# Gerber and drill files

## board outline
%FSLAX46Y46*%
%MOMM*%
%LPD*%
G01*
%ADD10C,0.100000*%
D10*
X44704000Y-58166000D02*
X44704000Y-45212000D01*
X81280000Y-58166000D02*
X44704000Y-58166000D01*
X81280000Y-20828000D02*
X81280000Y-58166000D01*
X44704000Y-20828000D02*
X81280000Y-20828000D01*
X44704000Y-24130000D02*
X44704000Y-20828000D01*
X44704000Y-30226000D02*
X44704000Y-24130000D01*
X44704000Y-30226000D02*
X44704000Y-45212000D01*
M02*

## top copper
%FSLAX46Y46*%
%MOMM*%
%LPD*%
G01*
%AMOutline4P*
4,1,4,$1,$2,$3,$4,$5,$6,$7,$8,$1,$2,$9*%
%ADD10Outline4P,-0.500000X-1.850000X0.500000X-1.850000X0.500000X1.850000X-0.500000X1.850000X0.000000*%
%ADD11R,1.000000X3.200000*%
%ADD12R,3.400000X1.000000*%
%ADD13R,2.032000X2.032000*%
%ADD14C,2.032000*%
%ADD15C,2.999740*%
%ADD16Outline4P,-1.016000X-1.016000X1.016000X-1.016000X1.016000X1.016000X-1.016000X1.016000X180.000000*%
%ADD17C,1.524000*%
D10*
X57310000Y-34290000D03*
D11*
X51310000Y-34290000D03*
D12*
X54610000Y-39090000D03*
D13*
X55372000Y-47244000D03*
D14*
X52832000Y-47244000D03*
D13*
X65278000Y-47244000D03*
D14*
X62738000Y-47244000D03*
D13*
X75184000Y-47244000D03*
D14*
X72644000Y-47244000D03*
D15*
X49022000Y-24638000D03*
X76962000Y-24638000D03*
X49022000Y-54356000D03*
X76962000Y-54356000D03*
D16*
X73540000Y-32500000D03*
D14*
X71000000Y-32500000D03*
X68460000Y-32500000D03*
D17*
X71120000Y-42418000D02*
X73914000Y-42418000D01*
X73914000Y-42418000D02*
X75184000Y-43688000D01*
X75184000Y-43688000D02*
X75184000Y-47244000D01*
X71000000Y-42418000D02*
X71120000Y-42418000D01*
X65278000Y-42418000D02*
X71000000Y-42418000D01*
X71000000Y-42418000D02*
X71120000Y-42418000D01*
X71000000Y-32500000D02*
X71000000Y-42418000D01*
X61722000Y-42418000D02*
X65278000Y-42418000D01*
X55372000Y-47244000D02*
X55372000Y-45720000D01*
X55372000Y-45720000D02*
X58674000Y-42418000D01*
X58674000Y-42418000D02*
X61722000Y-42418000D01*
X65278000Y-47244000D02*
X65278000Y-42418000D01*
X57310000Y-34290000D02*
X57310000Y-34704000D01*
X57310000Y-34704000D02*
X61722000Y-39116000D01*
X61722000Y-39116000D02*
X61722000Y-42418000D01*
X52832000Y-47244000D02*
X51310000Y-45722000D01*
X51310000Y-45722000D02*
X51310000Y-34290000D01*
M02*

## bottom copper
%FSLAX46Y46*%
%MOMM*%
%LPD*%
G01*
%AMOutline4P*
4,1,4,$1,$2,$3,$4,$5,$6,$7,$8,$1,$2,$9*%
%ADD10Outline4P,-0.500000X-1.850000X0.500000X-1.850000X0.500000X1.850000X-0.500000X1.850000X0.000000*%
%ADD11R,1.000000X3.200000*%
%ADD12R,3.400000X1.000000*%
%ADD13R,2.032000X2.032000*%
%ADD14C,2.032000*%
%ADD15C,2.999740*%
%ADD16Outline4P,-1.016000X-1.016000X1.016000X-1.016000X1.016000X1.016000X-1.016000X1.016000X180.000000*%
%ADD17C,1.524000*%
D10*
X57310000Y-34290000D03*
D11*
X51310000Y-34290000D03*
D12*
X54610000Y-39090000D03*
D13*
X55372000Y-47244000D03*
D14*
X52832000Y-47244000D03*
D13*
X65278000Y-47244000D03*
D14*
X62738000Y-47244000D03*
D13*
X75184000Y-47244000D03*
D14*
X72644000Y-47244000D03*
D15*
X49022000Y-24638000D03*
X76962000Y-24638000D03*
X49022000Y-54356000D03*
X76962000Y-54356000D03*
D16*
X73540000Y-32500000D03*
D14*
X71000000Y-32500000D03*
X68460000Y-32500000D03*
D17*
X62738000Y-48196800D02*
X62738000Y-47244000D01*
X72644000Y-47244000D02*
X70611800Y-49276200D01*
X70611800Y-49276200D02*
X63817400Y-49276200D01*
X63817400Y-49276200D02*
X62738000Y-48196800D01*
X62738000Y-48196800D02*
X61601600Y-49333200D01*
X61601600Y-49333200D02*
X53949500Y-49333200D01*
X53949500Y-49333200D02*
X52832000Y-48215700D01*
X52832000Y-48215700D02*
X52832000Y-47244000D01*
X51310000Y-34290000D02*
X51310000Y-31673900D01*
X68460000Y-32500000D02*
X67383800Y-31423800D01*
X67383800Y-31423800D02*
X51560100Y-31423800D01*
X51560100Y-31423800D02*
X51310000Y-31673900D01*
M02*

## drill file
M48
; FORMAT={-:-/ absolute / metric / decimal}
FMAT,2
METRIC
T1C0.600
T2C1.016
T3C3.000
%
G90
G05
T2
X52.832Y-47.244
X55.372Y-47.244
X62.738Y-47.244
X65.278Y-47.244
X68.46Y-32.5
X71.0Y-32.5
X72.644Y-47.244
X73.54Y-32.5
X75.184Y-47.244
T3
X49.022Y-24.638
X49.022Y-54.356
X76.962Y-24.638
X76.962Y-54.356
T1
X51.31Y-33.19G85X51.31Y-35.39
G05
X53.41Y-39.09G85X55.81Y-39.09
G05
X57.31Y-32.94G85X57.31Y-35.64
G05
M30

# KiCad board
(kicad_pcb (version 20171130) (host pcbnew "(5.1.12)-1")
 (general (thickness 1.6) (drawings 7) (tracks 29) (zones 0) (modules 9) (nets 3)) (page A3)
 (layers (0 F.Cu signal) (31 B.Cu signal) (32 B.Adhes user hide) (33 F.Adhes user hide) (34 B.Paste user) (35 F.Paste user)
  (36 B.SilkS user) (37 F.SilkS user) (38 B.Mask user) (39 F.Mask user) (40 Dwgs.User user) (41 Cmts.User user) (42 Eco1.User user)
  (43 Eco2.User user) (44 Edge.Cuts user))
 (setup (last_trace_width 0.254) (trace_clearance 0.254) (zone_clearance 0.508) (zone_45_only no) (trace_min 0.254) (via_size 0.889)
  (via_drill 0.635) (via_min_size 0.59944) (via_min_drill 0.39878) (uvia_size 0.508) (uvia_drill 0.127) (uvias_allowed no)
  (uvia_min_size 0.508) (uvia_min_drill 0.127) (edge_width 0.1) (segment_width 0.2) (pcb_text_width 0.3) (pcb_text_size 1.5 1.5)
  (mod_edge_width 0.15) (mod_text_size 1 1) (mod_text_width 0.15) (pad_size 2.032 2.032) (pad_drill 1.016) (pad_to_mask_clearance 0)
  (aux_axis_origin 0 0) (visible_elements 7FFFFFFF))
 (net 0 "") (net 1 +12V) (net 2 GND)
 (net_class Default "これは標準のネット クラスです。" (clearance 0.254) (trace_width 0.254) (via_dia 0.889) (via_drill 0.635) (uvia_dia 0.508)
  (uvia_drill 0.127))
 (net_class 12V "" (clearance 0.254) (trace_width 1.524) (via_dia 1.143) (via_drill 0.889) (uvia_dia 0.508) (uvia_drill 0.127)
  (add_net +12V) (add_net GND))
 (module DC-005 (layer F.Cu) (at 54.61 34.29)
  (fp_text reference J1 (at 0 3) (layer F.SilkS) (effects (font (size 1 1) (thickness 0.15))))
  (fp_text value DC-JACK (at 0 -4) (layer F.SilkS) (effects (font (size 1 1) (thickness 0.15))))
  (pad 1 thru_hole trapezoid (at 2.7 0) (size 1 3.7) (drill oval 0.6 3.3) (layers *.Cu *.Mask F.SilkS) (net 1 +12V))
  (pad 2 thru_hole rect (at -3.3 0) (size 1 3.2) (drill oval 0.6 2.8) (layers *.Cu *.Mask F.SilkS) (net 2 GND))
  (pad 3 thru_hole rect (at 0 4.8) (size 3.4 1) (drill oval 3 0.6) (layers *.Cu *.Mask F.SilkS)))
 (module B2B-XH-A (layer F.Cu) (at 54.102 47.244 180)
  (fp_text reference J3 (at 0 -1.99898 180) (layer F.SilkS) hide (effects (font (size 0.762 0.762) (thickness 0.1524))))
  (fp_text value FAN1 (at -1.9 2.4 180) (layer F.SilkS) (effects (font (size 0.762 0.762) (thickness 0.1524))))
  (pad 1 thru_hole rect (at -1.27 0 180) (size 2.032 2.032) (drill 1.016) (layers *.Cu *.Mask F.SilkS) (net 1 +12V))
  (pad 2 thru_hole circle (at 1.27 0 180) (size 2.032 2.032) (drill 1.016) (layers *.Cu *.Mask F.SilkS) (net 2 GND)))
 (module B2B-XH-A (layer F.Cu) (at 64.008 47.244 180)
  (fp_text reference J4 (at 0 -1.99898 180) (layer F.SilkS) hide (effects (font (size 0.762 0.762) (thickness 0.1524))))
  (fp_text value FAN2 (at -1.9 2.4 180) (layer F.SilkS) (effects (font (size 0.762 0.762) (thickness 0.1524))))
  (pad 1 thru_hole rect (at -1.27 0 180) (size 2.032 2.032) (drill 1.016) (layers *.Cu *.Mask F.SilkS) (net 1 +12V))
  (pad 2 thru_hole circle (at 1.27 0 180) (size 2.032 2.032) (drill 1.016) (layers *.Cu *.Mask F.SilkS) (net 2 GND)))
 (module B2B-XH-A (layer F.Cu) (at 73.914 47.244 180)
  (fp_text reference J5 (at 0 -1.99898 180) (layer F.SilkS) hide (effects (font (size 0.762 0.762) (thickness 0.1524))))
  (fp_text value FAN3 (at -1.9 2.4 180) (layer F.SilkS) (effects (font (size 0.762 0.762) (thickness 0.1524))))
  (pad 1 thru_hole rect (at -1.27 0 180) (size 2.032 2.032) (drill 1.016) (layers *.Cu *.Mask F.SilkS) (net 1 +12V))
  (pad 2 thru_hole circle (at 1.27 0 180) (size 2.032 2.032) (drill 1.016) (layers *.Cu *.Mask F.SilkS) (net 2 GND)))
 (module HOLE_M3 (layer F.Cu) (at 49.022 24.638)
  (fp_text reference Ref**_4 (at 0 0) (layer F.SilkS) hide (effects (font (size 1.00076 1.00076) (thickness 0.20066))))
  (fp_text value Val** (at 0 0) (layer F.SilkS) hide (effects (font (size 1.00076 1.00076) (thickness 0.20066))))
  (pad "" thru_hole circle (at 0 0) (size 2.99974 2.99974) (drill 2.99974) (layers *.Cu *.Mask F.SilkS) (clearance 1.50114)))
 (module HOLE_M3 (layer F.Cu) (at 76.962 24.638)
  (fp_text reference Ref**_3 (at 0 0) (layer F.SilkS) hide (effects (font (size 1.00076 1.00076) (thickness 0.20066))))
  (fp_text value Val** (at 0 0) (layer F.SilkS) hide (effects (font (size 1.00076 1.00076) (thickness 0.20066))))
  (pad "" thru_hole circle (at 0 0) (size 2.99974 2.99974) (drill 2.99974) (layers *.Cu *.Mask F.SilkS) (clearance 1.50114)))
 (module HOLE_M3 (layer F.Cu) (at 49.022 54.356)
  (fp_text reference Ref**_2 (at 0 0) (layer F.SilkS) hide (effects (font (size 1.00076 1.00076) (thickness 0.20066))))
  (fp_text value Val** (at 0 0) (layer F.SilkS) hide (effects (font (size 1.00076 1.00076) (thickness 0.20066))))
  (pad "" thru_hole circle (at 0 0) (size 2.99974 2.99974) (drill 2.99974) (layers *.Cu *.Mask F.SilkS) (clearance 1.50114)))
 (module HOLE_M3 (layer F.Cu) (at 76.962 54.356)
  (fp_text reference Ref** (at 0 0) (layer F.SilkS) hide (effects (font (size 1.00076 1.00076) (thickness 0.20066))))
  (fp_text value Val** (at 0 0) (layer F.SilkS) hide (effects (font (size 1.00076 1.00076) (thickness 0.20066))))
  (pad "" thru_hole circle (at 0 0) (size 2.99974 2.99974) (drill 2.99974) (layers *.Cu *.Mask F.SilkS) (clearance 1.50114)))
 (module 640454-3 (layer F.Cu) (at 71 32.5 180)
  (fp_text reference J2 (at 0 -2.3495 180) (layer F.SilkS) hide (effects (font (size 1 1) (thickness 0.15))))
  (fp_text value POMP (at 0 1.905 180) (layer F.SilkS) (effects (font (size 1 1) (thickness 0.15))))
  (pad 1 thru_hole trapezoid (at -2.54 0 180) (size 2.032 2.032) (drill 1.016) (layers *.Cu *.Mask F.SilkS))
  (pad 2 thru_hole circle (at 0 0 180) (size 2.032 2.032) (drill 1.016) (layers *.Cu *.Mask F.SilkS) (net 1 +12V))
  (pad 3 thru_hole circle (at 2.54 0 180) (size 2.032 2.032) (drill 1.016) (layers *.Cu *.Mask F.SilkS) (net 2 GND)))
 (gr_line (start 44.704 58.166) (end 44.704 45.212) (angle 90) (layer Edge.Cuts) (width 0.1))
 (gr_line (start 81.28 58.166) (end 44.704 58.166) (angle 90) (layer Edge.Cuts) (width 0.1))
 (gr_line (start 81.28 20.828) (end 81.28 58.166) (angle 90) (layer Edge.Cuts) (width 0.1))
 (gr_line (start 44.704 20.828) (end 81.28 20.828) (angle 90) (layer Edge.Cuts) (width 0.1))
 (gr_line (start 44.704 24.13) (end 44.704 20.828) (angle 90) (layer Edge.Cuts) (width 0.1))
 (gr_line (start 44.704 30.226) (end 44.704 24.13) (angle 90) (layer Edge.Cuts) (width 0.1))
 (gr_line (start 44.704 30.226) (end 44.704 45.212) (angle 90) (layer Edge.Cuts) (width 0.1))
 (segment (start 71.12 42.418) (end 73.914 42.418) (width 1.524) (layer F.Cu) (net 1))
 (segment (start 73.914 42.418) (end 75.184 43.688) (width 1.524) (layer F.Cu) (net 1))
 (segment (start 75.184 43.688) (end 75.184 47.244) (width 1.524) (layer F.Cu) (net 1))
 (segment (start 71 42.418) (end 71.12 42.418) (width 1.524) (layer F.Cu) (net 1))
 (segment (start 65.278 42.418) (end 71 42.418) (width 1.524) (layer F.Cu) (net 1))
 (segment (start 71 42.418) (end 71.12 42.418) (width 1.524) (layer F.Cu) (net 1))
 (segment (start 71 32.5) (end 71 42.418) (width 1.524) (layer F.Cu) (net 1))
 (segment (start 61.722 42.418) (end 65.278 42.418) (width 1.524) (layer F.Cu) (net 1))
 (segment (start 55.372 47.244) (end 55.372 45.72) (width 1.524) (layer F.Cu) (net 1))
 (segment (start 55.372 45.72) (end 58.674 42.418) (width 1.524) (layer F.Cu) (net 1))
 (segment (start 58.674 42.418) (end 61.722 42.418) (width 1.524) (layer F.Cu) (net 1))
 (segment (start 65.278 47.244) (end 65.278 42.418) (width 1.524) (layer F.Cu) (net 1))
 (segment (start 57.31 34.29) (end 57.31 34.704) (width 1.524) (layer F.Cu) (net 1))
 (segment (start 57.31 34.704) (end 61.722 39.116) (width 1.524) (layer F.Cu) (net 1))
 (segment (start 61.722 39.116) (end 61.722 42.418) (width 1.524) (layer F.Cu) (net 1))
 (segment (start 52.832 47.244) (end 51.31 45.722) (width 1.524) (layer F.Cu) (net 2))
 (segment (start 51.31 45.722) (end 51.31 34.29) (width 1.524) (layer F.Cu) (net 2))
 (segment (start 62.738 48.1968) (end 62.738 47.244) (width 1.524) (layer B.Cu) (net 2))
 (segment (start 72.644 47.244) (end 70.6118 49.2762) (width 1.524) (layer B.Cu) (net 2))
 (segment (start 70.6118 49.2762) (end 63.8174 49.2762) (width 1.524) (layer B.Cu) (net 2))
 (segment (start 63.8174 49.2762) (end 62.738 48.1968) (width 1.524) (layer B.Cu) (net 2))
 (segment (start 62.738 48.1968) (end 61.6016 49.3332) (width 1.524) (layer B.Cu) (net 2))
 (segment (start 61.6016 49.3332) (end 53.9495 49.3332) (width 1.524) (layer B.Cu) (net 2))
 (segment (start 53.9495 49.3332) (end 52.832 48.2157) (width 1.524) (layer B.Cu) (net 2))
 (segment (start 52.832 48.2157) (end 52.832 47.244) (width 1.524) (layer B.Cu) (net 2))
 (segment (start 51.31 34.29) (end 51.31 31.6739) (width 1.524) (layer B.Cu) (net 2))
 (segment (start 68.46 32.5) (end 67.3838 31.4238) (width 1.524) (layer B.Cu) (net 2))
 (segment (start 67.3838 31.4238) (end 51.5601 31.4238) (width 1.524) (layer B.Cu) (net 2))
 (segment (start 51.5601 31.4238) (end 51.31 31.6739) (width 1.524) (layer B.Cu) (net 2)))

